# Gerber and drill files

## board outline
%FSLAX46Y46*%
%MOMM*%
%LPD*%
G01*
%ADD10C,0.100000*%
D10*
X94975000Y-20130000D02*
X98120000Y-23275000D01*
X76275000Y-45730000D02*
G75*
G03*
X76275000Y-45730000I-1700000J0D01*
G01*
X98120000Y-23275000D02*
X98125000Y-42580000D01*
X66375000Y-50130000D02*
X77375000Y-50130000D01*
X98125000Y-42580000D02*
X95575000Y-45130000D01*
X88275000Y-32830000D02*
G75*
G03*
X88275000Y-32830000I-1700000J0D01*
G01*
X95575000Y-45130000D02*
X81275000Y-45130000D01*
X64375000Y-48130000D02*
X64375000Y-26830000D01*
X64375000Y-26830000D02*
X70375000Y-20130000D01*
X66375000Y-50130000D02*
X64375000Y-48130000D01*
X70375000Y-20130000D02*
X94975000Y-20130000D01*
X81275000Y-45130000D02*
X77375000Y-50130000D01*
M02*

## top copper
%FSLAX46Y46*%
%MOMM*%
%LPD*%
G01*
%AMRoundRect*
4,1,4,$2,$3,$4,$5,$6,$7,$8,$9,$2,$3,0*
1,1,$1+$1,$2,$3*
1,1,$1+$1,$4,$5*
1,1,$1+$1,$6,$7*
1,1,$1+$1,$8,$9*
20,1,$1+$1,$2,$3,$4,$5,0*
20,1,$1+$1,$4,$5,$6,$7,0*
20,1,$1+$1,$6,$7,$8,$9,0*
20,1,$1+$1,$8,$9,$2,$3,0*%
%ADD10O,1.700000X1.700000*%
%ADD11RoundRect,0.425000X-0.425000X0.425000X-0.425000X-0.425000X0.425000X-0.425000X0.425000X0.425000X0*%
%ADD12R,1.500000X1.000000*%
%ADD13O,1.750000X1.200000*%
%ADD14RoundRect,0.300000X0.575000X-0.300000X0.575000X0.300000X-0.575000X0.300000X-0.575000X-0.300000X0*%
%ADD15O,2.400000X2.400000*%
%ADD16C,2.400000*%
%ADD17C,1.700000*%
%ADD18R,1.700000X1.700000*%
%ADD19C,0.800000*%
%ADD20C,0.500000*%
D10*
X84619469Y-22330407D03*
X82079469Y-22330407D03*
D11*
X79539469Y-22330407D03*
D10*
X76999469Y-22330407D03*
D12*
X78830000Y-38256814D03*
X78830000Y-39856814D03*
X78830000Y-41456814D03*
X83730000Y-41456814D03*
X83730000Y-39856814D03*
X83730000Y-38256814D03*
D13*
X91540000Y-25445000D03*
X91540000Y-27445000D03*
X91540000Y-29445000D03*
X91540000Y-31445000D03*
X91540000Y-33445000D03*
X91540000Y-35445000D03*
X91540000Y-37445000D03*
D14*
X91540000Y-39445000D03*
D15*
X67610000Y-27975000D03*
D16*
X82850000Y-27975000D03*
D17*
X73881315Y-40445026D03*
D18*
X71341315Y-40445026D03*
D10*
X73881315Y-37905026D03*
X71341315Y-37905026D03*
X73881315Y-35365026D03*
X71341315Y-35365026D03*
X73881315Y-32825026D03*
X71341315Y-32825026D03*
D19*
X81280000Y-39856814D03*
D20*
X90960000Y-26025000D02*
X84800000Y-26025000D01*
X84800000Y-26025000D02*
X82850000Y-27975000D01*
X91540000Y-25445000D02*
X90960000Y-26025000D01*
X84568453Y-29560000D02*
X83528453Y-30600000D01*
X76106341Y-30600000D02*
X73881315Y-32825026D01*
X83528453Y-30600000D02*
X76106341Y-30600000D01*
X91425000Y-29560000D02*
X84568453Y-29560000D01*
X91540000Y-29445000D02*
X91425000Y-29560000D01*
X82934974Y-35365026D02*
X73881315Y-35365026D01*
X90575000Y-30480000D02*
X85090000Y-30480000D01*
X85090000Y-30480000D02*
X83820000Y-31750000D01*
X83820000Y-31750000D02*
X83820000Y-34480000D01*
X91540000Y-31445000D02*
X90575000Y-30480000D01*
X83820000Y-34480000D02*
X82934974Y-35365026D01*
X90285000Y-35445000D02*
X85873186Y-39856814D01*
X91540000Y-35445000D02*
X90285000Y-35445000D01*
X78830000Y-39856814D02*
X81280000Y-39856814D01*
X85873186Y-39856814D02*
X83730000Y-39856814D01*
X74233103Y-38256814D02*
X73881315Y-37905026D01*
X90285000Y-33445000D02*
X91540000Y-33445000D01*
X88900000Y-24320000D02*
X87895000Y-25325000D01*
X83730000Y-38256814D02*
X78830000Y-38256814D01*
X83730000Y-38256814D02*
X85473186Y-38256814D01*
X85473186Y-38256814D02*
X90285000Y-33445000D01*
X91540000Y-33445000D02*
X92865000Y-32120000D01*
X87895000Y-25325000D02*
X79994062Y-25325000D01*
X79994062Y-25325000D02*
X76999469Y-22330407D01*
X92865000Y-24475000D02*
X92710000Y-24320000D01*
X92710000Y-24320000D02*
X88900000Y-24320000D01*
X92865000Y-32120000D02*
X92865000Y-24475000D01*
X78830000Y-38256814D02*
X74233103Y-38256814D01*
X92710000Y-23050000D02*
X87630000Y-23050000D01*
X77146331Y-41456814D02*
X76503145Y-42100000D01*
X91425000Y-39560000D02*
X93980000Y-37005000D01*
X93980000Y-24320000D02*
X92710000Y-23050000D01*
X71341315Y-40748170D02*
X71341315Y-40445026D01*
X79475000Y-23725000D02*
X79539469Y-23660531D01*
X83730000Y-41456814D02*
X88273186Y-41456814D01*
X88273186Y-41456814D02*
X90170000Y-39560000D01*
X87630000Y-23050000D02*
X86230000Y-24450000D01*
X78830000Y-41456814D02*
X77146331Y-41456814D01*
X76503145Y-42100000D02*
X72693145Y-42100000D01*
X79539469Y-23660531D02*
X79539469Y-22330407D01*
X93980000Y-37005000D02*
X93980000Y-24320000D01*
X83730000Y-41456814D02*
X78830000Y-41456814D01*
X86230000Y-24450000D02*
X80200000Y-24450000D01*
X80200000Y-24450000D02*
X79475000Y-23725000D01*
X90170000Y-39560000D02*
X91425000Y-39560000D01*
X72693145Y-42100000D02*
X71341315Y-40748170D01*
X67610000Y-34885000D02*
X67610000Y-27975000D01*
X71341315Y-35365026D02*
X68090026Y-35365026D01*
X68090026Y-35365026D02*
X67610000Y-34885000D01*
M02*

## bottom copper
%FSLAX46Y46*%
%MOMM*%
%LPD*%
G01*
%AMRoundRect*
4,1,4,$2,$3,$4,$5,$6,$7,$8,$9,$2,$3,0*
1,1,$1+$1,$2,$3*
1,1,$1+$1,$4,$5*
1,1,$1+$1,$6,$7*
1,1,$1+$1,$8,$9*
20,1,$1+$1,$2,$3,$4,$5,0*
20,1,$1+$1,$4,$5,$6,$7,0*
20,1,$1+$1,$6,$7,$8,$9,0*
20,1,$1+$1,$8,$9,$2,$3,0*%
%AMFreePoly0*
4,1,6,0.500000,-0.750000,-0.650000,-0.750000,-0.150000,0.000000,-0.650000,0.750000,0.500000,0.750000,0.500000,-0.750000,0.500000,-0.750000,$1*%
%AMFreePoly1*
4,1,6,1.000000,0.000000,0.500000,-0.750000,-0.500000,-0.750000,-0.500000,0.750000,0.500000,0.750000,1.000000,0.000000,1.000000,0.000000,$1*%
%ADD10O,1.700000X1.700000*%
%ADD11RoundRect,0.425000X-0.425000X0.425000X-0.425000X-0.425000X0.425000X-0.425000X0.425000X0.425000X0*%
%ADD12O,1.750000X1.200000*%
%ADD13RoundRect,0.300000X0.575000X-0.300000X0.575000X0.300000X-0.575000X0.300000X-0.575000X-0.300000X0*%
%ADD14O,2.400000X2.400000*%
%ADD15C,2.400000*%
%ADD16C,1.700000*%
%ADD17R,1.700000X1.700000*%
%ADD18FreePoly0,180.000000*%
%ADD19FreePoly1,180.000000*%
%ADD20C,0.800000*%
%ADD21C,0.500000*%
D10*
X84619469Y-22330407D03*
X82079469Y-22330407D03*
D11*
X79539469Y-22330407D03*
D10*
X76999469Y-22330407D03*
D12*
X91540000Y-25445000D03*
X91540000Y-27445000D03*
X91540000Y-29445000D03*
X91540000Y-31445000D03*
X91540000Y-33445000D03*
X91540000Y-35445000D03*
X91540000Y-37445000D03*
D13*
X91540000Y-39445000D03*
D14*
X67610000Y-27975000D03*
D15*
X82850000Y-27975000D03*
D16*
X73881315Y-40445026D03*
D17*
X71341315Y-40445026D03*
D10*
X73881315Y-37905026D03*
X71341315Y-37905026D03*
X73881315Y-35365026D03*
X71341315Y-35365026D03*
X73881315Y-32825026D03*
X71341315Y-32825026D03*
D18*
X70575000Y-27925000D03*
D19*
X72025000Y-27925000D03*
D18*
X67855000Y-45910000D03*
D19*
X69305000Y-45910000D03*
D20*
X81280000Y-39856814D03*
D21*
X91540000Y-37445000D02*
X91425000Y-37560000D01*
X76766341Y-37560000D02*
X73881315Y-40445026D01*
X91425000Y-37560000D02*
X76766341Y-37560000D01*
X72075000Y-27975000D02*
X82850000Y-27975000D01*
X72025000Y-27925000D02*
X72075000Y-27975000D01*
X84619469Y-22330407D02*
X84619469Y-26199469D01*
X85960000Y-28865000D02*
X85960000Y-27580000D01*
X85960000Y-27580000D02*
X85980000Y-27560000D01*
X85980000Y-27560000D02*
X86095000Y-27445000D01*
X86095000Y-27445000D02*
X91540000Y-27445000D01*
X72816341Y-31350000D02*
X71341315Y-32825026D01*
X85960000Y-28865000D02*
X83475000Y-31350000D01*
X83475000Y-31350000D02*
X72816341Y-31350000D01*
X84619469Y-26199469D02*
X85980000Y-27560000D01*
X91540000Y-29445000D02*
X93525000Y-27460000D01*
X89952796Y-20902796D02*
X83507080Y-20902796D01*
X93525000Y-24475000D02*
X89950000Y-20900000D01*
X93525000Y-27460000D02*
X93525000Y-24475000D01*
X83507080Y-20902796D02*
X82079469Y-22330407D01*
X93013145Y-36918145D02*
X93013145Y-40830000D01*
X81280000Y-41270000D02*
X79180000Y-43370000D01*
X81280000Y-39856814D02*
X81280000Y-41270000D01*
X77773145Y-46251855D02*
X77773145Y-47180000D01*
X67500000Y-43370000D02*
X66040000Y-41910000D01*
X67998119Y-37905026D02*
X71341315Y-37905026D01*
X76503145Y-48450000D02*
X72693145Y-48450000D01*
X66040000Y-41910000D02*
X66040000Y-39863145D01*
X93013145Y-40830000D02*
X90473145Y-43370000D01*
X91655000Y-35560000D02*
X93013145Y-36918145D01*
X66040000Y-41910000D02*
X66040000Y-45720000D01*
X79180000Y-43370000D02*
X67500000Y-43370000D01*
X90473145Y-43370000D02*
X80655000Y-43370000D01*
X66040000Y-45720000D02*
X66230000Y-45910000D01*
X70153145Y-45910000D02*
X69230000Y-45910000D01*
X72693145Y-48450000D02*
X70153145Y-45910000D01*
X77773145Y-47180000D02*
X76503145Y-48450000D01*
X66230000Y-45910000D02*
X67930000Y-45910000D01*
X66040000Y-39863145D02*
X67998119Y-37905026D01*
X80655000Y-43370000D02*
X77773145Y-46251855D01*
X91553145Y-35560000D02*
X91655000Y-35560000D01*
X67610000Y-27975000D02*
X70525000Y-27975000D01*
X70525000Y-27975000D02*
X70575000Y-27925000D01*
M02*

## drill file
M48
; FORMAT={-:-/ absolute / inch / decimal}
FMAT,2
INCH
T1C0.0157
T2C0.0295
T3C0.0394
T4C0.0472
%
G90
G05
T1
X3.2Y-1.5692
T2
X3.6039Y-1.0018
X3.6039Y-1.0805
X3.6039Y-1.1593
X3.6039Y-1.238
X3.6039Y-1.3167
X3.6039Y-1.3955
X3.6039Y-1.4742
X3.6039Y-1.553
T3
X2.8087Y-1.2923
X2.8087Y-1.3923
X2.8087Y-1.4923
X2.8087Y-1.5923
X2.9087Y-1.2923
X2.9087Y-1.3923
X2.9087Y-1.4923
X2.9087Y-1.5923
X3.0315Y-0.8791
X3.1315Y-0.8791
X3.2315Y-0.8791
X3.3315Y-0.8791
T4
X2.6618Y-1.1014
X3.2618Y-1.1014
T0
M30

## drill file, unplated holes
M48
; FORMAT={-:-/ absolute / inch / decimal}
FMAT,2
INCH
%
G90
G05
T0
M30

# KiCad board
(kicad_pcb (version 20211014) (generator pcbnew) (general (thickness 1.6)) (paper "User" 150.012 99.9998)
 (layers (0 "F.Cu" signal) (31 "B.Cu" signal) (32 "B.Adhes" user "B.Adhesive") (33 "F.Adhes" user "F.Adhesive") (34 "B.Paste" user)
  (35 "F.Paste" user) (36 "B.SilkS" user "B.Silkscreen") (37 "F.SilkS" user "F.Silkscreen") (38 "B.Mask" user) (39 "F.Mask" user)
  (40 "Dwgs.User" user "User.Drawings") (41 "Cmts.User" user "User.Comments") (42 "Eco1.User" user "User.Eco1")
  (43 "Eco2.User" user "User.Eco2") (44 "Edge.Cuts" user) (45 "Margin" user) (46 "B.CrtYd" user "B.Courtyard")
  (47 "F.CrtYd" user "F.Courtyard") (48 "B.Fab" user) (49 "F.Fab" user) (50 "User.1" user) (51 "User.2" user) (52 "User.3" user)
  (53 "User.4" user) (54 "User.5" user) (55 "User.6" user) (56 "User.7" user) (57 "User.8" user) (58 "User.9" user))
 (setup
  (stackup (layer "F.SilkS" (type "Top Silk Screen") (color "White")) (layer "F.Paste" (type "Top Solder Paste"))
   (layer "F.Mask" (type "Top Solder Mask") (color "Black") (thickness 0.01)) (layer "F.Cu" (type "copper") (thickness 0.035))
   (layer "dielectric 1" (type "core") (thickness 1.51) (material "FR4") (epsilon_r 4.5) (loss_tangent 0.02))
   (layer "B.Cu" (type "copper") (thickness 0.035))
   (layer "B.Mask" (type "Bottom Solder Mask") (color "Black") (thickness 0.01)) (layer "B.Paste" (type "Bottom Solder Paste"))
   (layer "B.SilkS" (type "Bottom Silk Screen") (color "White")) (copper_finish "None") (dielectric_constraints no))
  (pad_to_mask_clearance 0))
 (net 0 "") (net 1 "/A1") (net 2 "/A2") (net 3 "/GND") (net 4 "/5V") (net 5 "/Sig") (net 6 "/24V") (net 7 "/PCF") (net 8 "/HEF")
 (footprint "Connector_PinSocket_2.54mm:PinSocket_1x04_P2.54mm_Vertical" (layer "F.Cu") (at 84.619469 22.330407 -90)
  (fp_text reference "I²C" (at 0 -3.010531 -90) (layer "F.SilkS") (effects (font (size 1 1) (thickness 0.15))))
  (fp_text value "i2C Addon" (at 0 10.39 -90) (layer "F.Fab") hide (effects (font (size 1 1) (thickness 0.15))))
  (pad "1" thru_hole oval (at 0 0 270) (size 1.7 1.7) (drill 1) (layers *.Cu *.Mask) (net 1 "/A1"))
  (pad "2" thru_hole oval (at 0 2.54 270) (size 1.7 1.7) (drill 1) (layers *.Cu *.Mask) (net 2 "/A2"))
  (pad "3" thru_hole roundrect (at 0 5.08 270) (size 1.7 1.7) (drill 1) (layers *.Cu *.Mask) (roundrect_rratio 0.25) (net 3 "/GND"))
  (pad "4" thru_hole oval (at 0 7.62 270) (size 1.7 1.7) (drill 1) (layers *.Cu *.Mask) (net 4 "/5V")))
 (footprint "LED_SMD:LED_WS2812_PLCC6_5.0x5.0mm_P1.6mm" (layer "F.Cu") (at 81.28 39.856814)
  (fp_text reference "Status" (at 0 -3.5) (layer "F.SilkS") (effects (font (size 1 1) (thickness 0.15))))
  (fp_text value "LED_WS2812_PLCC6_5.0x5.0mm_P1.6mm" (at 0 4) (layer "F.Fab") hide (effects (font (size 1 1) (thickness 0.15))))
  (pad "1" smd rect (at 2.45 -1.6) (size 1.5 1) (layers "F.Cu" "F.Paste" "F.Mask") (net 4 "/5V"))
  (pad "2" smd rect (at 2.45 0) (size 1.5 1) (layers "F.Cu" "F.Paste" "F.Mask") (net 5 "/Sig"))
  (pad "3" smd rect (at 2.45 1.6) (size 1.5 1) (layers "F.Cu" "F.Paste" "F.Mask") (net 3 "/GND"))
  (pad "4" smd rect (at -2.45 1.6) (size 1.5 1) (layers "F.Cu" "F.Paste" "F.Mask") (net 3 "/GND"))
  (pad "5" smd rect (at -2.45 0) (size 1.5 1) (layers "F.Cu" "F.Paste" "F.Mask") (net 5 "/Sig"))
  (pad "6" smd rect (at -2.45 -1.6) (size 1.5 1) (layers "F.Cu" "F.Paste" "F.Mask") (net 4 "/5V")))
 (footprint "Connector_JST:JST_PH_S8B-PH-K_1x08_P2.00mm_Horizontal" (layer "F.Cu") (at 91.54 39.445 90)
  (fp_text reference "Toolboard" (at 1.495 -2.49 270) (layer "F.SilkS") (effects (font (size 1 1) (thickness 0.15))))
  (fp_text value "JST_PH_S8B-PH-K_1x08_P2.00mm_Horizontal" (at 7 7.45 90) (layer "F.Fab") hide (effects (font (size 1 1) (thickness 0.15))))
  (pad "1" thru_hole roundrect (at 0 0 90) (size 1.2 1.75) (drill 0.75) (layers *.Cu *.Mask) (roundrect_rratio 0.25) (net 3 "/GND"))
  (pad "2" thru_hole oval (at 2 0 90) (size 1.2 1.75) (drill 0.75) (layers *.Cu *.Mask) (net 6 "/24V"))
  (pad "3" thru_hole oval (at 4 0 90) (size 1.2 1.75) (drill 0.75) (layers *.Cu *.Mask) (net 5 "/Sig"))
  (pad "4" thru_hole oval (at 6 0 90) (size 1.2 1.75) (drill 0.75) (layers *.Cu *.Mask) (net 4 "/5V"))
  (pad "5" thru_hole oval (at 8 0 90) (size 1.2 1.75) (drill 0.75) (layers *.Cu *.Mask) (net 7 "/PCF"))
  (pad "6" thru_hole oval (at 10 0 90) (size 1.2 1.75) (drill 0.75) (layers *.Cu *.Mask) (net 2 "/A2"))
  (pad "7" thru_hole oval (at 12 0 90) (size 1.2 1.75) (drill 0.75) (layers *.Cu *.Mask) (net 1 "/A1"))
  (pad "8" thru_hole oval (at 14 0 90) (size 1.2 1.75) (drill 0.75) (layers *.Cu *.Mask) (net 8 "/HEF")))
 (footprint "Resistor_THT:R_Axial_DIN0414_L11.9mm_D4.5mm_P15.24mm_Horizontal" (layer "F.Cu") (at 82.85 27.975 180)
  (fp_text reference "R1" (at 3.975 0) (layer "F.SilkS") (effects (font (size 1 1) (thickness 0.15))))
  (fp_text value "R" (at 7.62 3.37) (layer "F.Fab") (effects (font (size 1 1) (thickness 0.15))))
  (pad "1" thru_hole circle (at 0 0 180) (size 2.4 2.4) (drill 1.2) (layers *.Cu *.Mask) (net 8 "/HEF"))
  (pad "2" thru_hole oval (at 15.24 0 180) (size 2.4 2.4) (drill 1.2) (layers *.Cu *.Mask) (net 8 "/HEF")))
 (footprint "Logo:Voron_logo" (layer "F.Cu") (at 80.775 32.73)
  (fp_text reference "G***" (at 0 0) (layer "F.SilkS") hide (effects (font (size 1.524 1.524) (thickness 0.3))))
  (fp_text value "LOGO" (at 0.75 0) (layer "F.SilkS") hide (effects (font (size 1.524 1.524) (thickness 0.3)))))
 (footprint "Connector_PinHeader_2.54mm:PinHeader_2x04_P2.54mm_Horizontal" (layer "F.Cu") (at 63.261315 32.825026)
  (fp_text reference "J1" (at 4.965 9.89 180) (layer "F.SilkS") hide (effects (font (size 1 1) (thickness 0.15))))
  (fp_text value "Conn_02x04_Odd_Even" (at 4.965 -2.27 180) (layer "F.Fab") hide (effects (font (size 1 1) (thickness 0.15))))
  (pad "1" thru_hole oval (at 8.08 0 180) (size 1.7 1.7) (drill 1) (layers *.Cu *.Mask) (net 1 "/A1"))
  (pad "2" thru_hole oval (at 10.62 0 180) (size 1.7 1.7) (drill 1) (layers *.Cu *.Mask) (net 2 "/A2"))
  (pad "3" thru_hole oval (at 8.08 2.54 180) (size 1.7 1.7) (drill 1) (layers *.Cu *.Mask) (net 8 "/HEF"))
  (pad "4" thru_hole oval (at 10.62 2.54 180) (size 1.7 1.7) (drill 1) (layers *.Cu *.Mask) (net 7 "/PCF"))
  (pad "5" thru_hole oval (at 8.08 5.08 180) (size 1.7 1.7) (drill 1) (layers *.Cu *.Mask) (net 5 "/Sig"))
  (pad "6" thru_hole oval (at 10.62 5.08 180) (size 1.7 1.7) (drill 1) (layers *.Cu *.Mask) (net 4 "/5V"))
  (pad "7" thru_hole rect (at 8.08 7.62 180) (size 1.7 1.7) (drill 1) (layers *.Cu *.Mask) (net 3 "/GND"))
  (pad "8" thru_hole circle (at 10.62 7.62 180) (size 1.7 1.7) (drill 1) (layers *.Cu *.Mask) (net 6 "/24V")))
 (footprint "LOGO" (layer "F.Cu") (at 93.98 21.59)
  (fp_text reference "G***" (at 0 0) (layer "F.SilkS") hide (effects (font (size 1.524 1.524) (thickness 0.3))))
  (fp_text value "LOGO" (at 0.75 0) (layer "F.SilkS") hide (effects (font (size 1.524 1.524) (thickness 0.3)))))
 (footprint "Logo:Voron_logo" (layer "B.Cu") (at 80.775 32.73 180)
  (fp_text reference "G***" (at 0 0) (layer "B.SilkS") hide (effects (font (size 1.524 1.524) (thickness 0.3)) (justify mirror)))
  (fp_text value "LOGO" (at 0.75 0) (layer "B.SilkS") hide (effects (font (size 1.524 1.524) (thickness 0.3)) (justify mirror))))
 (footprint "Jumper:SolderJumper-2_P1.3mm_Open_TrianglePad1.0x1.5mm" (layer "B.Cu") (at 71.3 27.925 180)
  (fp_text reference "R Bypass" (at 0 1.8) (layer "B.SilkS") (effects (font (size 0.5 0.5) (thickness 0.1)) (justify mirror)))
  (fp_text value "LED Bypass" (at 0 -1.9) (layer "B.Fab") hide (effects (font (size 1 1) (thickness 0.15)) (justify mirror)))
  (pad "1" smd custom (at -0.725 0 180) (size 0.3 0.3) (layers "B.Cu" "B.Mask") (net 8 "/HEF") (zone_connect 2)
   (options (clearance outline) (anchor rect)) (primitives))
  (pad "2" smd custom (at 0.725 0 180) (size 0.3 0.3) (layers "B.Cu" "B.Mask") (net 8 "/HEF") (zone_connect 2)
   (options (clearance outline) (anchor rect)) (primitives)))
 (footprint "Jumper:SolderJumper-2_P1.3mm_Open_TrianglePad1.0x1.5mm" (layer "B.Cu") (at 68.58 45.91 180)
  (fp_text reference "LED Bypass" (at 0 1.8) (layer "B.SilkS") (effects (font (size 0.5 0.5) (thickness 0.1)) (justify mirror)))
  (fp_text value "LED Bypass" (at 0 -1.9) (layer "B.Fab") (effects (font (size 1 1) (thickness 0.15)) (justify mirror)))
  (pad "1" smd custom (at -0.725 0 180) (size 0.3 0.3) (layers "B.Cu" "B.Mask") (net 5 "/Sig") (zone_connect 2)
   (options (clearance outline) (anchor rect)) (primitives))
  (pad "2" smd custom (at 0.725 0 180) (size 0.3 0.3) (layers "B.Cu" "B.Mask") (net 5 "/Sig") (zone_connect 2)
   (options (clearance outline) (anchor rect)) (primitives)))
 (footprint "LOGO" (layer "B.Cu") (at 71.12 22.86 180)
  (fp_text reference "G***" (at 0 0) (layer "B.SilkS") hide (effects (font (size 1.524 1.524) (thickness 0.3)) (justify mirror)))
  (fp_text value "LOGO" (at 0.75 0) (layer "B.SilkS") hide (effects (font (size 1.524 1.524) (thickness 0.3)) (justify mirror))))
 (gr_line (start 94.975 20.13) (end 98.12 23.275) (layer "Edge.Cuts") (width 0.1))
 (gr_circle (center 74.575 45.73) (end 76.275 45.73) (layer "Edge.Cuts") (width 0.1) (fill none))
 (gr_line (start 98.12 23.275) (end 98.125 42.58) (layer "Edge.Cuts") (width 0.1))
 (gr_line (start 66.375 50.13) (end 77.375 50.13) (layer "Edge.Cuts") (width 0.1))
 (gr_line (start 98.125 42.58) (end 95.575 45.13) (layer "Edge.Cuts") (width 0.1))
 (gr_circle (center 86.575 32.83) (end 88.275 32.83) (layer "Edge.Cuts") (width 0.1) (fill none))
 (gr_line (start 95.575 45.13) (end 81.275 45.13) (layer "Edge.Cuts") (width 0.1))
 (gr_line (start 64.375 48.13) (end 64.375 26.83) (layer "Edge.Cuts") (width 0.1))
 (gr_line (start 64.375 26.83) (end 70.375 20.13) (layer "Edge.Cuts") (width 0.1))
 (gr_line (start 66.375 50.13) (end 64.375 48.13) (layer "Edge.Cuts") (width 0.1))
 (gr_line (start 70.375 20.13) (end 94.975 20.13) (layer "Edge.Cuts") (width 0.1))
 (gr_line (start 81.275 45.13) (end 77.375 50.13) (layer "Edge.Cuts") (width 0.1))
 (segment (start 91.54 37.445) (end 91.425 37.56) (width 0.5) (layer "B.Cu") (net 6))
 (segment (start 76.766341 37.56) (end 73.881315 40.445026) (width 0.5) (layer "B.Cu") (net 6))
 (segment (start 91.425 37.56) (end 76.766341 37.56) (width 0.5) (layer "B.Cu") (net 6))
 (segment (start 67.61 34.885) (end 67.61 27.975) (width 0.5) (layer "F.Cu") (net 8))
 (segment (start 90.96 26.025) (end 84.8 26.025) (width 0.5) (layer "F.Cu") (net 8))
 (segment (start 84.8 26.025) (end 82.85 27.975) (width 0.5) (layer "F.Cu") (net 8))
 (segment (start 91.54 25.445) (end 90.96 26.025) (width 0.5) (layer "F.Cu") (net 8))
 (segment (start 71.341315 35.365026) (end 68.090026 35.365026) (width 0.5) (layer "F.Cu") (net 8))
 (segment (start 68.090026 35.365026) (end 67.61 34.885) (width 0.5) (layer "F.Cu") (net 8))
 (segment (start 72.075 27.975) (end 82.85 27.975) (width 0.5) (layer "B.Cu") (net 8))
 (segment (start 72.025 27.925) (end 72.075 27.975) (width 0.5) (layer "B.Cu") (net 8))
 (segment (start 67.61 27.975) (end 70.525 27.975) (width 0.5) (layer "B.Cu") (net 8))
 (segment (start 70.525 27.975) (end 70.575 27.925) (width 0.5) (layer "B.Cu") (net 8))
 (segment (start 84.619469 22.330407) (end 84.619469 26.199469) (width 0.5) (layer "B.Cu") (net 1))
 (segment (start 85.96 28.865) (end 85.96 27.58) (width 0.5) (layer "B.Cu") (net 1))
 (segment (start 85.96 27.58) (end 85.98 27.56) (width 0.5) (layer "B.Cu") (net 1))
 (segment (start 85.98 27.56) (end 86.095 27.445) (width 0.5) (layer "B.Cu") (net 1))
 (segment (start 86.095 27.445) (end 91.54 27.445) (width 0.5) (layer "B.Cu") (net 1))
 (segment (start 72.816341 31.35) (end 71.341315 32.825026) (width 0.5) (layer "B.Cu") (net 1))
 (segment (start 85.96 28.865) (end 83.475 31.35) (width 0.5) (layer "B.Cu") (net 1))
 (segment (start 83.475 31.35) (end 72.816341 31.35) (width 0.5) (layer "B.Cu") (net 1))
 (segment (start 84.619469 26.199469) (end 85.98 27.56) (width 0.5) (layer "B.Cu") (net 1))
 (segment (start 84.568453 29.56) (end 83.528453 30.6) (width 0.5) (layer "F.Cu") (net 2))
 (segment (start 76.106341 30.6) (end 73.881315 32.825026) (width 0.5) (layer "F.Cu") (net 2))
 (segment (start 83.528453 30.6) (end 76.106341 30.6) (width 0.5) (layer "F.Cu") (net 2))
 (segment (start 91.425 29.56) (end 84.568453 29.56) (width 0.5) (layer "F.Cu") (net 2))
 (segment (start 91.54 29.445) (end 91.425 29.56) (width 0.5) (layer "F.Cu") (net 2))
 (segment (start 91.54 29.445) (end 93.525 27.46) (width 0.5) (layer "B.Cu") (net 2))
 (segment (start 89.952796 20.902796) (end 83.50708 20.902796) (width 0.5) (layer "B.Cu") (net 2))
 (segment (start 93.525 24.475) (end 89.95 20.9) (width 0.5) (layer "B.Cu") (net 2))
 (segment (start 93.525 27.46) (end 93.525 24.475) (width 0.5) (layer "B.Cu") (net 2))
 (segment (start 83.50708 20.902796) (end 82.079469 22.330407) (width 0.5) (layer "B.Cu") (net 2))
 (segment (start 82.934974 35.365026) (end 73.881315 35.365026) (width 0.5) (layer "F.Cu") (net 7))
 (segment (start 90.575 30.48) (end 85.09 30.48) (width 0.5) (layer "F.Cu") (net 7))
 (segment (start 85.09 30.48) (end 83.82 31.75) (width 0.5) (layer "F.Cu") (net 7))
 (segment (start 83.82 31.75) (end 83.82 34.48) (width 0.5) (layer "F.Cu") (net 7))
 (segment (start 91.54 31.445) (end 90.575 30.48) (width 0.5) (layer "F.Cu") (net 7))
 (segment (start 83.82 34.48) (end 82.934974 35.365026) (width 0.5) (layer "F.Cu") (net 7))
 (segment (start 90.285 35.445) (end 85.873186 39.856814) (width 0.5) (layer "F.Cu") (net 5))
 (segment (start 91.54 35.445) (end 90.285 35.445) (width 0.5) (layer "F.Cu") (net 5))
 (segment (start 78.83 39.856814) (end 81.28 39.856814) (width 0.5) (layer "F.Cu") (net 5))
 (segment (start 85.873186 39.856814) (end 83.73 39.856814) (width 0.5) (layer "F.Cu") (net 5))
 (via blind (at 81.28 39.856814) (size 0.8) (drill 0.4) (layers "F.Cu" "B.Cu") (free) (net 5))
 (segment (start 93.013145 36.918145) (end 93.013145 40.83) (width 0.5) (layer "B.Cu") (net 5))
 (segment (start 81.28 41.27) (end 79.18 43.37) (width 0.5) (layer "B.Cu") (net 5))
 (segment (start 81.28 39.856814) (end 81.28 41.27) (width 0.5) (layer "B.Cu") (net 5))
 (segment (start 77.773145 46.251855) (end 77.773145 47.18) (width 0.5) (layer "B.Cu") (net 5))
 (segment (start 67.5 43.37) (end 66.04 41.91) (width 0.5) (layer "B.Cu") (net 5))
 (segment (start 67.998119 37.905026) (end 71.341315 37.905026) (width 0.5) (layer "B.Cu") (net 5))
 (segment (start 76.503145 48.45) (end 72.693145 48.45) (width 0.5) (layer "B.Cu") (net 5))
 (segment (start 66.04 41.91) (end 66.04 39.863145) (width 0.5) (layer "B.Cu") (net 5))
 (segment (start 93.013145 40.83) (end 90.473145 43.37) (width 0.5) (layer "B.Cu") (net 5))
 (segment (start 91.655 35.56) (end 93.013145 36.918145) (width 0.5) (layer "B.Cu") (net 5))
 (segment (start 66.04 41.91) (end 66.04 45.72) (width 0.5) (layer "B.Cu") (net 5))
 (segment (start 79.18 43.37) (end 67.5 43.37) (width 0.5) (layer "B.Cu") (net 5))
 (segment (start 90.473145 43.37) (end 80.655 43.37) (width 0.5) (layer "B.Cu") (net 5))
 (segment (start 66.04 45.72) (end 66.23 45.91) (width 0.5) (layer "B.Cu") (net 5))
 (segment (start 70.153145 45.91) (end 69.23 45.91) (width 0.5) (layer "B.Cu") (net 5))
 (segment (start 72.693145 48.45) (end 70.153145 45.91) (width 0.5) (layer "B.Cu") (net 5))
 (segment (start 77.773145 47.18) (end 76.503145 48.45) (width 0.5) (layer "B.Cu") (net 5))
 (segment (start 66.23 45.91) (end 67.93 45.91) (width 0.5) (layer "B.Cu") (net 5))
 (segment (start 66.04 39.863145) (end 67.998119 37.905026) (width 0.5) (layer "B.Cu") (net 5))
 (segment (start 80.655 43.37) (end 77.773145 46.251855) (width 0.5) (layer "B.Cu") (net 5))
 (segment (start 91.553145 35.56) (end 91.655 35.56) (width 0.5) (layer "B.Cu") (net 5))
 (segment (start 74.233103 38.256814) (end 73.881315 37.905026) (width 0.5) (layer "F.Cu") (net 4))
 (segment (start 90.285 33.445) (end 91.54 33.445) (width 0.5) (layer "F.Cu") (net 4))
 (segment (start 88.9 24.32) (end 87.895 25.325) (width 0.5) (layer "F.Cu") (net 4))
 (segment (start 83.73 38.256814) (end 78.83 38.256814) (width 0.5) (layer "F.Cu") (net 4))
 (segment (start 83.73 38.256814) (end 85.473186 38.256814) (width 0.5) (layer "F.Cu") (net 4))
 (segment (start 85.473186 38.256814) (end 90.285 33.445) (width 0.5) (layer "F.Cu") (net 4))
 (segment (start 91.54 33.445) (end 92.865 32.12) (width 0.5) (layer "F.Cu") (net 4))
 (segment (start 87.895 25.325) (end 79.994062 25.325) (width 0.5) (layer "F.Cu") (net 4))
 (segment (start 79.994062 25.325) (end 76.999469 22.330407) (width 0.5) (layer "F.Cu") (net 4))
 (segment (start 92.865 24.475) (end 92.71 24.32) (width 0.5) (layer "F.Cu") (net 4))
 (segment (start 92.71 24.32) (end 88.9 24.32) (width 0.5) (layer "F.Cu") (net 4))
 (segment (start 92.865 32.12) (end 92.865 24.475) (width 0.5) (layer "F.Cu") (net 4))
 (segment (start 78.83 38.256814) (end 74.233103 38.256814) (width 0.5) (layer "F.Cu") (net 4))
 (segment (start 92.71 23.05) (end 87.63 23.05) (width 0.5) (layer "F.Cu") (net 3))
 (segment (start 77.146331 41.456814) (end 76.503145 42.1) (width 0.5) (layer "F.Cu") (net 3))
 (segment (start 91.425 39.56) (end 93.98 37.005) (width 0.5) (layer "F.Cu") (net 3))
 (segment (start 93.98 24.32) (end 92.71 23.05) (width 0.5) (layer "F.Cu") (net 3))
 (segment (start 71.341315 40.74817) (end 71.341315 40.445026) (width 0.5) (layer "F.Cu") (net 3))
 (segment (start 79.475 23.725) (end 79.539469 23.660531) (width 0.5) (layer "F.Cu") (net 3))
 (segment (start 83.73 41.456814) (end 88.273186 41.456814) (width 0.5) (layer "F.Cu") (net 3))
 (segment (start 88.273186 41.456814) (end 90.17 39.56) (width 0.5) (layer "F.Cu") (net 3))
 (segment (start 87.63 23.05) (end 86.23 24.45) (width 0.5) (layer "F.Cu") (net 3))
 (segment (start 78.83 41.456814) (end 77.146331 41.456814) (width 0.5) (layer "F.Cu") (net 3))
 (segment (start 76.503145 42.1) (end 72.693145 42.1) (width 0.5) (layer "F.Cu") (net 3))
 (segment (start 79.539469 23.660531) (end 79.539469 22.330407) (width 0.5) (layer "F.Cu") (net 3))
 (segment (start 93.98 37.005) (end 93.98 24.32) (width 0.5) (layer "F.Cu") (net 3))
 (segment (start 83.73 41.456814) (end 78.83 41.456814) (width 0.5) (layer "F.Cu") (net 3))
 (segment (start 86.23 24.45) (end 80.2 24.45) (width 0.5) (layer "F.Cu") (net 3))
 (segment (start 80.2 24.45) (end 79.475 23.725) (width 0.5) (layer "F.Cu") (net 3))
 (segment (start 90.17 39.56) (end 91.425 39.56) (width 0.5) (layer "F.Cu") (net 3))
 (segment (start 72.693145 42.1) (end 71.341315 40.74817) (width 0.5) (layer "F.Cu") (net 3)))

